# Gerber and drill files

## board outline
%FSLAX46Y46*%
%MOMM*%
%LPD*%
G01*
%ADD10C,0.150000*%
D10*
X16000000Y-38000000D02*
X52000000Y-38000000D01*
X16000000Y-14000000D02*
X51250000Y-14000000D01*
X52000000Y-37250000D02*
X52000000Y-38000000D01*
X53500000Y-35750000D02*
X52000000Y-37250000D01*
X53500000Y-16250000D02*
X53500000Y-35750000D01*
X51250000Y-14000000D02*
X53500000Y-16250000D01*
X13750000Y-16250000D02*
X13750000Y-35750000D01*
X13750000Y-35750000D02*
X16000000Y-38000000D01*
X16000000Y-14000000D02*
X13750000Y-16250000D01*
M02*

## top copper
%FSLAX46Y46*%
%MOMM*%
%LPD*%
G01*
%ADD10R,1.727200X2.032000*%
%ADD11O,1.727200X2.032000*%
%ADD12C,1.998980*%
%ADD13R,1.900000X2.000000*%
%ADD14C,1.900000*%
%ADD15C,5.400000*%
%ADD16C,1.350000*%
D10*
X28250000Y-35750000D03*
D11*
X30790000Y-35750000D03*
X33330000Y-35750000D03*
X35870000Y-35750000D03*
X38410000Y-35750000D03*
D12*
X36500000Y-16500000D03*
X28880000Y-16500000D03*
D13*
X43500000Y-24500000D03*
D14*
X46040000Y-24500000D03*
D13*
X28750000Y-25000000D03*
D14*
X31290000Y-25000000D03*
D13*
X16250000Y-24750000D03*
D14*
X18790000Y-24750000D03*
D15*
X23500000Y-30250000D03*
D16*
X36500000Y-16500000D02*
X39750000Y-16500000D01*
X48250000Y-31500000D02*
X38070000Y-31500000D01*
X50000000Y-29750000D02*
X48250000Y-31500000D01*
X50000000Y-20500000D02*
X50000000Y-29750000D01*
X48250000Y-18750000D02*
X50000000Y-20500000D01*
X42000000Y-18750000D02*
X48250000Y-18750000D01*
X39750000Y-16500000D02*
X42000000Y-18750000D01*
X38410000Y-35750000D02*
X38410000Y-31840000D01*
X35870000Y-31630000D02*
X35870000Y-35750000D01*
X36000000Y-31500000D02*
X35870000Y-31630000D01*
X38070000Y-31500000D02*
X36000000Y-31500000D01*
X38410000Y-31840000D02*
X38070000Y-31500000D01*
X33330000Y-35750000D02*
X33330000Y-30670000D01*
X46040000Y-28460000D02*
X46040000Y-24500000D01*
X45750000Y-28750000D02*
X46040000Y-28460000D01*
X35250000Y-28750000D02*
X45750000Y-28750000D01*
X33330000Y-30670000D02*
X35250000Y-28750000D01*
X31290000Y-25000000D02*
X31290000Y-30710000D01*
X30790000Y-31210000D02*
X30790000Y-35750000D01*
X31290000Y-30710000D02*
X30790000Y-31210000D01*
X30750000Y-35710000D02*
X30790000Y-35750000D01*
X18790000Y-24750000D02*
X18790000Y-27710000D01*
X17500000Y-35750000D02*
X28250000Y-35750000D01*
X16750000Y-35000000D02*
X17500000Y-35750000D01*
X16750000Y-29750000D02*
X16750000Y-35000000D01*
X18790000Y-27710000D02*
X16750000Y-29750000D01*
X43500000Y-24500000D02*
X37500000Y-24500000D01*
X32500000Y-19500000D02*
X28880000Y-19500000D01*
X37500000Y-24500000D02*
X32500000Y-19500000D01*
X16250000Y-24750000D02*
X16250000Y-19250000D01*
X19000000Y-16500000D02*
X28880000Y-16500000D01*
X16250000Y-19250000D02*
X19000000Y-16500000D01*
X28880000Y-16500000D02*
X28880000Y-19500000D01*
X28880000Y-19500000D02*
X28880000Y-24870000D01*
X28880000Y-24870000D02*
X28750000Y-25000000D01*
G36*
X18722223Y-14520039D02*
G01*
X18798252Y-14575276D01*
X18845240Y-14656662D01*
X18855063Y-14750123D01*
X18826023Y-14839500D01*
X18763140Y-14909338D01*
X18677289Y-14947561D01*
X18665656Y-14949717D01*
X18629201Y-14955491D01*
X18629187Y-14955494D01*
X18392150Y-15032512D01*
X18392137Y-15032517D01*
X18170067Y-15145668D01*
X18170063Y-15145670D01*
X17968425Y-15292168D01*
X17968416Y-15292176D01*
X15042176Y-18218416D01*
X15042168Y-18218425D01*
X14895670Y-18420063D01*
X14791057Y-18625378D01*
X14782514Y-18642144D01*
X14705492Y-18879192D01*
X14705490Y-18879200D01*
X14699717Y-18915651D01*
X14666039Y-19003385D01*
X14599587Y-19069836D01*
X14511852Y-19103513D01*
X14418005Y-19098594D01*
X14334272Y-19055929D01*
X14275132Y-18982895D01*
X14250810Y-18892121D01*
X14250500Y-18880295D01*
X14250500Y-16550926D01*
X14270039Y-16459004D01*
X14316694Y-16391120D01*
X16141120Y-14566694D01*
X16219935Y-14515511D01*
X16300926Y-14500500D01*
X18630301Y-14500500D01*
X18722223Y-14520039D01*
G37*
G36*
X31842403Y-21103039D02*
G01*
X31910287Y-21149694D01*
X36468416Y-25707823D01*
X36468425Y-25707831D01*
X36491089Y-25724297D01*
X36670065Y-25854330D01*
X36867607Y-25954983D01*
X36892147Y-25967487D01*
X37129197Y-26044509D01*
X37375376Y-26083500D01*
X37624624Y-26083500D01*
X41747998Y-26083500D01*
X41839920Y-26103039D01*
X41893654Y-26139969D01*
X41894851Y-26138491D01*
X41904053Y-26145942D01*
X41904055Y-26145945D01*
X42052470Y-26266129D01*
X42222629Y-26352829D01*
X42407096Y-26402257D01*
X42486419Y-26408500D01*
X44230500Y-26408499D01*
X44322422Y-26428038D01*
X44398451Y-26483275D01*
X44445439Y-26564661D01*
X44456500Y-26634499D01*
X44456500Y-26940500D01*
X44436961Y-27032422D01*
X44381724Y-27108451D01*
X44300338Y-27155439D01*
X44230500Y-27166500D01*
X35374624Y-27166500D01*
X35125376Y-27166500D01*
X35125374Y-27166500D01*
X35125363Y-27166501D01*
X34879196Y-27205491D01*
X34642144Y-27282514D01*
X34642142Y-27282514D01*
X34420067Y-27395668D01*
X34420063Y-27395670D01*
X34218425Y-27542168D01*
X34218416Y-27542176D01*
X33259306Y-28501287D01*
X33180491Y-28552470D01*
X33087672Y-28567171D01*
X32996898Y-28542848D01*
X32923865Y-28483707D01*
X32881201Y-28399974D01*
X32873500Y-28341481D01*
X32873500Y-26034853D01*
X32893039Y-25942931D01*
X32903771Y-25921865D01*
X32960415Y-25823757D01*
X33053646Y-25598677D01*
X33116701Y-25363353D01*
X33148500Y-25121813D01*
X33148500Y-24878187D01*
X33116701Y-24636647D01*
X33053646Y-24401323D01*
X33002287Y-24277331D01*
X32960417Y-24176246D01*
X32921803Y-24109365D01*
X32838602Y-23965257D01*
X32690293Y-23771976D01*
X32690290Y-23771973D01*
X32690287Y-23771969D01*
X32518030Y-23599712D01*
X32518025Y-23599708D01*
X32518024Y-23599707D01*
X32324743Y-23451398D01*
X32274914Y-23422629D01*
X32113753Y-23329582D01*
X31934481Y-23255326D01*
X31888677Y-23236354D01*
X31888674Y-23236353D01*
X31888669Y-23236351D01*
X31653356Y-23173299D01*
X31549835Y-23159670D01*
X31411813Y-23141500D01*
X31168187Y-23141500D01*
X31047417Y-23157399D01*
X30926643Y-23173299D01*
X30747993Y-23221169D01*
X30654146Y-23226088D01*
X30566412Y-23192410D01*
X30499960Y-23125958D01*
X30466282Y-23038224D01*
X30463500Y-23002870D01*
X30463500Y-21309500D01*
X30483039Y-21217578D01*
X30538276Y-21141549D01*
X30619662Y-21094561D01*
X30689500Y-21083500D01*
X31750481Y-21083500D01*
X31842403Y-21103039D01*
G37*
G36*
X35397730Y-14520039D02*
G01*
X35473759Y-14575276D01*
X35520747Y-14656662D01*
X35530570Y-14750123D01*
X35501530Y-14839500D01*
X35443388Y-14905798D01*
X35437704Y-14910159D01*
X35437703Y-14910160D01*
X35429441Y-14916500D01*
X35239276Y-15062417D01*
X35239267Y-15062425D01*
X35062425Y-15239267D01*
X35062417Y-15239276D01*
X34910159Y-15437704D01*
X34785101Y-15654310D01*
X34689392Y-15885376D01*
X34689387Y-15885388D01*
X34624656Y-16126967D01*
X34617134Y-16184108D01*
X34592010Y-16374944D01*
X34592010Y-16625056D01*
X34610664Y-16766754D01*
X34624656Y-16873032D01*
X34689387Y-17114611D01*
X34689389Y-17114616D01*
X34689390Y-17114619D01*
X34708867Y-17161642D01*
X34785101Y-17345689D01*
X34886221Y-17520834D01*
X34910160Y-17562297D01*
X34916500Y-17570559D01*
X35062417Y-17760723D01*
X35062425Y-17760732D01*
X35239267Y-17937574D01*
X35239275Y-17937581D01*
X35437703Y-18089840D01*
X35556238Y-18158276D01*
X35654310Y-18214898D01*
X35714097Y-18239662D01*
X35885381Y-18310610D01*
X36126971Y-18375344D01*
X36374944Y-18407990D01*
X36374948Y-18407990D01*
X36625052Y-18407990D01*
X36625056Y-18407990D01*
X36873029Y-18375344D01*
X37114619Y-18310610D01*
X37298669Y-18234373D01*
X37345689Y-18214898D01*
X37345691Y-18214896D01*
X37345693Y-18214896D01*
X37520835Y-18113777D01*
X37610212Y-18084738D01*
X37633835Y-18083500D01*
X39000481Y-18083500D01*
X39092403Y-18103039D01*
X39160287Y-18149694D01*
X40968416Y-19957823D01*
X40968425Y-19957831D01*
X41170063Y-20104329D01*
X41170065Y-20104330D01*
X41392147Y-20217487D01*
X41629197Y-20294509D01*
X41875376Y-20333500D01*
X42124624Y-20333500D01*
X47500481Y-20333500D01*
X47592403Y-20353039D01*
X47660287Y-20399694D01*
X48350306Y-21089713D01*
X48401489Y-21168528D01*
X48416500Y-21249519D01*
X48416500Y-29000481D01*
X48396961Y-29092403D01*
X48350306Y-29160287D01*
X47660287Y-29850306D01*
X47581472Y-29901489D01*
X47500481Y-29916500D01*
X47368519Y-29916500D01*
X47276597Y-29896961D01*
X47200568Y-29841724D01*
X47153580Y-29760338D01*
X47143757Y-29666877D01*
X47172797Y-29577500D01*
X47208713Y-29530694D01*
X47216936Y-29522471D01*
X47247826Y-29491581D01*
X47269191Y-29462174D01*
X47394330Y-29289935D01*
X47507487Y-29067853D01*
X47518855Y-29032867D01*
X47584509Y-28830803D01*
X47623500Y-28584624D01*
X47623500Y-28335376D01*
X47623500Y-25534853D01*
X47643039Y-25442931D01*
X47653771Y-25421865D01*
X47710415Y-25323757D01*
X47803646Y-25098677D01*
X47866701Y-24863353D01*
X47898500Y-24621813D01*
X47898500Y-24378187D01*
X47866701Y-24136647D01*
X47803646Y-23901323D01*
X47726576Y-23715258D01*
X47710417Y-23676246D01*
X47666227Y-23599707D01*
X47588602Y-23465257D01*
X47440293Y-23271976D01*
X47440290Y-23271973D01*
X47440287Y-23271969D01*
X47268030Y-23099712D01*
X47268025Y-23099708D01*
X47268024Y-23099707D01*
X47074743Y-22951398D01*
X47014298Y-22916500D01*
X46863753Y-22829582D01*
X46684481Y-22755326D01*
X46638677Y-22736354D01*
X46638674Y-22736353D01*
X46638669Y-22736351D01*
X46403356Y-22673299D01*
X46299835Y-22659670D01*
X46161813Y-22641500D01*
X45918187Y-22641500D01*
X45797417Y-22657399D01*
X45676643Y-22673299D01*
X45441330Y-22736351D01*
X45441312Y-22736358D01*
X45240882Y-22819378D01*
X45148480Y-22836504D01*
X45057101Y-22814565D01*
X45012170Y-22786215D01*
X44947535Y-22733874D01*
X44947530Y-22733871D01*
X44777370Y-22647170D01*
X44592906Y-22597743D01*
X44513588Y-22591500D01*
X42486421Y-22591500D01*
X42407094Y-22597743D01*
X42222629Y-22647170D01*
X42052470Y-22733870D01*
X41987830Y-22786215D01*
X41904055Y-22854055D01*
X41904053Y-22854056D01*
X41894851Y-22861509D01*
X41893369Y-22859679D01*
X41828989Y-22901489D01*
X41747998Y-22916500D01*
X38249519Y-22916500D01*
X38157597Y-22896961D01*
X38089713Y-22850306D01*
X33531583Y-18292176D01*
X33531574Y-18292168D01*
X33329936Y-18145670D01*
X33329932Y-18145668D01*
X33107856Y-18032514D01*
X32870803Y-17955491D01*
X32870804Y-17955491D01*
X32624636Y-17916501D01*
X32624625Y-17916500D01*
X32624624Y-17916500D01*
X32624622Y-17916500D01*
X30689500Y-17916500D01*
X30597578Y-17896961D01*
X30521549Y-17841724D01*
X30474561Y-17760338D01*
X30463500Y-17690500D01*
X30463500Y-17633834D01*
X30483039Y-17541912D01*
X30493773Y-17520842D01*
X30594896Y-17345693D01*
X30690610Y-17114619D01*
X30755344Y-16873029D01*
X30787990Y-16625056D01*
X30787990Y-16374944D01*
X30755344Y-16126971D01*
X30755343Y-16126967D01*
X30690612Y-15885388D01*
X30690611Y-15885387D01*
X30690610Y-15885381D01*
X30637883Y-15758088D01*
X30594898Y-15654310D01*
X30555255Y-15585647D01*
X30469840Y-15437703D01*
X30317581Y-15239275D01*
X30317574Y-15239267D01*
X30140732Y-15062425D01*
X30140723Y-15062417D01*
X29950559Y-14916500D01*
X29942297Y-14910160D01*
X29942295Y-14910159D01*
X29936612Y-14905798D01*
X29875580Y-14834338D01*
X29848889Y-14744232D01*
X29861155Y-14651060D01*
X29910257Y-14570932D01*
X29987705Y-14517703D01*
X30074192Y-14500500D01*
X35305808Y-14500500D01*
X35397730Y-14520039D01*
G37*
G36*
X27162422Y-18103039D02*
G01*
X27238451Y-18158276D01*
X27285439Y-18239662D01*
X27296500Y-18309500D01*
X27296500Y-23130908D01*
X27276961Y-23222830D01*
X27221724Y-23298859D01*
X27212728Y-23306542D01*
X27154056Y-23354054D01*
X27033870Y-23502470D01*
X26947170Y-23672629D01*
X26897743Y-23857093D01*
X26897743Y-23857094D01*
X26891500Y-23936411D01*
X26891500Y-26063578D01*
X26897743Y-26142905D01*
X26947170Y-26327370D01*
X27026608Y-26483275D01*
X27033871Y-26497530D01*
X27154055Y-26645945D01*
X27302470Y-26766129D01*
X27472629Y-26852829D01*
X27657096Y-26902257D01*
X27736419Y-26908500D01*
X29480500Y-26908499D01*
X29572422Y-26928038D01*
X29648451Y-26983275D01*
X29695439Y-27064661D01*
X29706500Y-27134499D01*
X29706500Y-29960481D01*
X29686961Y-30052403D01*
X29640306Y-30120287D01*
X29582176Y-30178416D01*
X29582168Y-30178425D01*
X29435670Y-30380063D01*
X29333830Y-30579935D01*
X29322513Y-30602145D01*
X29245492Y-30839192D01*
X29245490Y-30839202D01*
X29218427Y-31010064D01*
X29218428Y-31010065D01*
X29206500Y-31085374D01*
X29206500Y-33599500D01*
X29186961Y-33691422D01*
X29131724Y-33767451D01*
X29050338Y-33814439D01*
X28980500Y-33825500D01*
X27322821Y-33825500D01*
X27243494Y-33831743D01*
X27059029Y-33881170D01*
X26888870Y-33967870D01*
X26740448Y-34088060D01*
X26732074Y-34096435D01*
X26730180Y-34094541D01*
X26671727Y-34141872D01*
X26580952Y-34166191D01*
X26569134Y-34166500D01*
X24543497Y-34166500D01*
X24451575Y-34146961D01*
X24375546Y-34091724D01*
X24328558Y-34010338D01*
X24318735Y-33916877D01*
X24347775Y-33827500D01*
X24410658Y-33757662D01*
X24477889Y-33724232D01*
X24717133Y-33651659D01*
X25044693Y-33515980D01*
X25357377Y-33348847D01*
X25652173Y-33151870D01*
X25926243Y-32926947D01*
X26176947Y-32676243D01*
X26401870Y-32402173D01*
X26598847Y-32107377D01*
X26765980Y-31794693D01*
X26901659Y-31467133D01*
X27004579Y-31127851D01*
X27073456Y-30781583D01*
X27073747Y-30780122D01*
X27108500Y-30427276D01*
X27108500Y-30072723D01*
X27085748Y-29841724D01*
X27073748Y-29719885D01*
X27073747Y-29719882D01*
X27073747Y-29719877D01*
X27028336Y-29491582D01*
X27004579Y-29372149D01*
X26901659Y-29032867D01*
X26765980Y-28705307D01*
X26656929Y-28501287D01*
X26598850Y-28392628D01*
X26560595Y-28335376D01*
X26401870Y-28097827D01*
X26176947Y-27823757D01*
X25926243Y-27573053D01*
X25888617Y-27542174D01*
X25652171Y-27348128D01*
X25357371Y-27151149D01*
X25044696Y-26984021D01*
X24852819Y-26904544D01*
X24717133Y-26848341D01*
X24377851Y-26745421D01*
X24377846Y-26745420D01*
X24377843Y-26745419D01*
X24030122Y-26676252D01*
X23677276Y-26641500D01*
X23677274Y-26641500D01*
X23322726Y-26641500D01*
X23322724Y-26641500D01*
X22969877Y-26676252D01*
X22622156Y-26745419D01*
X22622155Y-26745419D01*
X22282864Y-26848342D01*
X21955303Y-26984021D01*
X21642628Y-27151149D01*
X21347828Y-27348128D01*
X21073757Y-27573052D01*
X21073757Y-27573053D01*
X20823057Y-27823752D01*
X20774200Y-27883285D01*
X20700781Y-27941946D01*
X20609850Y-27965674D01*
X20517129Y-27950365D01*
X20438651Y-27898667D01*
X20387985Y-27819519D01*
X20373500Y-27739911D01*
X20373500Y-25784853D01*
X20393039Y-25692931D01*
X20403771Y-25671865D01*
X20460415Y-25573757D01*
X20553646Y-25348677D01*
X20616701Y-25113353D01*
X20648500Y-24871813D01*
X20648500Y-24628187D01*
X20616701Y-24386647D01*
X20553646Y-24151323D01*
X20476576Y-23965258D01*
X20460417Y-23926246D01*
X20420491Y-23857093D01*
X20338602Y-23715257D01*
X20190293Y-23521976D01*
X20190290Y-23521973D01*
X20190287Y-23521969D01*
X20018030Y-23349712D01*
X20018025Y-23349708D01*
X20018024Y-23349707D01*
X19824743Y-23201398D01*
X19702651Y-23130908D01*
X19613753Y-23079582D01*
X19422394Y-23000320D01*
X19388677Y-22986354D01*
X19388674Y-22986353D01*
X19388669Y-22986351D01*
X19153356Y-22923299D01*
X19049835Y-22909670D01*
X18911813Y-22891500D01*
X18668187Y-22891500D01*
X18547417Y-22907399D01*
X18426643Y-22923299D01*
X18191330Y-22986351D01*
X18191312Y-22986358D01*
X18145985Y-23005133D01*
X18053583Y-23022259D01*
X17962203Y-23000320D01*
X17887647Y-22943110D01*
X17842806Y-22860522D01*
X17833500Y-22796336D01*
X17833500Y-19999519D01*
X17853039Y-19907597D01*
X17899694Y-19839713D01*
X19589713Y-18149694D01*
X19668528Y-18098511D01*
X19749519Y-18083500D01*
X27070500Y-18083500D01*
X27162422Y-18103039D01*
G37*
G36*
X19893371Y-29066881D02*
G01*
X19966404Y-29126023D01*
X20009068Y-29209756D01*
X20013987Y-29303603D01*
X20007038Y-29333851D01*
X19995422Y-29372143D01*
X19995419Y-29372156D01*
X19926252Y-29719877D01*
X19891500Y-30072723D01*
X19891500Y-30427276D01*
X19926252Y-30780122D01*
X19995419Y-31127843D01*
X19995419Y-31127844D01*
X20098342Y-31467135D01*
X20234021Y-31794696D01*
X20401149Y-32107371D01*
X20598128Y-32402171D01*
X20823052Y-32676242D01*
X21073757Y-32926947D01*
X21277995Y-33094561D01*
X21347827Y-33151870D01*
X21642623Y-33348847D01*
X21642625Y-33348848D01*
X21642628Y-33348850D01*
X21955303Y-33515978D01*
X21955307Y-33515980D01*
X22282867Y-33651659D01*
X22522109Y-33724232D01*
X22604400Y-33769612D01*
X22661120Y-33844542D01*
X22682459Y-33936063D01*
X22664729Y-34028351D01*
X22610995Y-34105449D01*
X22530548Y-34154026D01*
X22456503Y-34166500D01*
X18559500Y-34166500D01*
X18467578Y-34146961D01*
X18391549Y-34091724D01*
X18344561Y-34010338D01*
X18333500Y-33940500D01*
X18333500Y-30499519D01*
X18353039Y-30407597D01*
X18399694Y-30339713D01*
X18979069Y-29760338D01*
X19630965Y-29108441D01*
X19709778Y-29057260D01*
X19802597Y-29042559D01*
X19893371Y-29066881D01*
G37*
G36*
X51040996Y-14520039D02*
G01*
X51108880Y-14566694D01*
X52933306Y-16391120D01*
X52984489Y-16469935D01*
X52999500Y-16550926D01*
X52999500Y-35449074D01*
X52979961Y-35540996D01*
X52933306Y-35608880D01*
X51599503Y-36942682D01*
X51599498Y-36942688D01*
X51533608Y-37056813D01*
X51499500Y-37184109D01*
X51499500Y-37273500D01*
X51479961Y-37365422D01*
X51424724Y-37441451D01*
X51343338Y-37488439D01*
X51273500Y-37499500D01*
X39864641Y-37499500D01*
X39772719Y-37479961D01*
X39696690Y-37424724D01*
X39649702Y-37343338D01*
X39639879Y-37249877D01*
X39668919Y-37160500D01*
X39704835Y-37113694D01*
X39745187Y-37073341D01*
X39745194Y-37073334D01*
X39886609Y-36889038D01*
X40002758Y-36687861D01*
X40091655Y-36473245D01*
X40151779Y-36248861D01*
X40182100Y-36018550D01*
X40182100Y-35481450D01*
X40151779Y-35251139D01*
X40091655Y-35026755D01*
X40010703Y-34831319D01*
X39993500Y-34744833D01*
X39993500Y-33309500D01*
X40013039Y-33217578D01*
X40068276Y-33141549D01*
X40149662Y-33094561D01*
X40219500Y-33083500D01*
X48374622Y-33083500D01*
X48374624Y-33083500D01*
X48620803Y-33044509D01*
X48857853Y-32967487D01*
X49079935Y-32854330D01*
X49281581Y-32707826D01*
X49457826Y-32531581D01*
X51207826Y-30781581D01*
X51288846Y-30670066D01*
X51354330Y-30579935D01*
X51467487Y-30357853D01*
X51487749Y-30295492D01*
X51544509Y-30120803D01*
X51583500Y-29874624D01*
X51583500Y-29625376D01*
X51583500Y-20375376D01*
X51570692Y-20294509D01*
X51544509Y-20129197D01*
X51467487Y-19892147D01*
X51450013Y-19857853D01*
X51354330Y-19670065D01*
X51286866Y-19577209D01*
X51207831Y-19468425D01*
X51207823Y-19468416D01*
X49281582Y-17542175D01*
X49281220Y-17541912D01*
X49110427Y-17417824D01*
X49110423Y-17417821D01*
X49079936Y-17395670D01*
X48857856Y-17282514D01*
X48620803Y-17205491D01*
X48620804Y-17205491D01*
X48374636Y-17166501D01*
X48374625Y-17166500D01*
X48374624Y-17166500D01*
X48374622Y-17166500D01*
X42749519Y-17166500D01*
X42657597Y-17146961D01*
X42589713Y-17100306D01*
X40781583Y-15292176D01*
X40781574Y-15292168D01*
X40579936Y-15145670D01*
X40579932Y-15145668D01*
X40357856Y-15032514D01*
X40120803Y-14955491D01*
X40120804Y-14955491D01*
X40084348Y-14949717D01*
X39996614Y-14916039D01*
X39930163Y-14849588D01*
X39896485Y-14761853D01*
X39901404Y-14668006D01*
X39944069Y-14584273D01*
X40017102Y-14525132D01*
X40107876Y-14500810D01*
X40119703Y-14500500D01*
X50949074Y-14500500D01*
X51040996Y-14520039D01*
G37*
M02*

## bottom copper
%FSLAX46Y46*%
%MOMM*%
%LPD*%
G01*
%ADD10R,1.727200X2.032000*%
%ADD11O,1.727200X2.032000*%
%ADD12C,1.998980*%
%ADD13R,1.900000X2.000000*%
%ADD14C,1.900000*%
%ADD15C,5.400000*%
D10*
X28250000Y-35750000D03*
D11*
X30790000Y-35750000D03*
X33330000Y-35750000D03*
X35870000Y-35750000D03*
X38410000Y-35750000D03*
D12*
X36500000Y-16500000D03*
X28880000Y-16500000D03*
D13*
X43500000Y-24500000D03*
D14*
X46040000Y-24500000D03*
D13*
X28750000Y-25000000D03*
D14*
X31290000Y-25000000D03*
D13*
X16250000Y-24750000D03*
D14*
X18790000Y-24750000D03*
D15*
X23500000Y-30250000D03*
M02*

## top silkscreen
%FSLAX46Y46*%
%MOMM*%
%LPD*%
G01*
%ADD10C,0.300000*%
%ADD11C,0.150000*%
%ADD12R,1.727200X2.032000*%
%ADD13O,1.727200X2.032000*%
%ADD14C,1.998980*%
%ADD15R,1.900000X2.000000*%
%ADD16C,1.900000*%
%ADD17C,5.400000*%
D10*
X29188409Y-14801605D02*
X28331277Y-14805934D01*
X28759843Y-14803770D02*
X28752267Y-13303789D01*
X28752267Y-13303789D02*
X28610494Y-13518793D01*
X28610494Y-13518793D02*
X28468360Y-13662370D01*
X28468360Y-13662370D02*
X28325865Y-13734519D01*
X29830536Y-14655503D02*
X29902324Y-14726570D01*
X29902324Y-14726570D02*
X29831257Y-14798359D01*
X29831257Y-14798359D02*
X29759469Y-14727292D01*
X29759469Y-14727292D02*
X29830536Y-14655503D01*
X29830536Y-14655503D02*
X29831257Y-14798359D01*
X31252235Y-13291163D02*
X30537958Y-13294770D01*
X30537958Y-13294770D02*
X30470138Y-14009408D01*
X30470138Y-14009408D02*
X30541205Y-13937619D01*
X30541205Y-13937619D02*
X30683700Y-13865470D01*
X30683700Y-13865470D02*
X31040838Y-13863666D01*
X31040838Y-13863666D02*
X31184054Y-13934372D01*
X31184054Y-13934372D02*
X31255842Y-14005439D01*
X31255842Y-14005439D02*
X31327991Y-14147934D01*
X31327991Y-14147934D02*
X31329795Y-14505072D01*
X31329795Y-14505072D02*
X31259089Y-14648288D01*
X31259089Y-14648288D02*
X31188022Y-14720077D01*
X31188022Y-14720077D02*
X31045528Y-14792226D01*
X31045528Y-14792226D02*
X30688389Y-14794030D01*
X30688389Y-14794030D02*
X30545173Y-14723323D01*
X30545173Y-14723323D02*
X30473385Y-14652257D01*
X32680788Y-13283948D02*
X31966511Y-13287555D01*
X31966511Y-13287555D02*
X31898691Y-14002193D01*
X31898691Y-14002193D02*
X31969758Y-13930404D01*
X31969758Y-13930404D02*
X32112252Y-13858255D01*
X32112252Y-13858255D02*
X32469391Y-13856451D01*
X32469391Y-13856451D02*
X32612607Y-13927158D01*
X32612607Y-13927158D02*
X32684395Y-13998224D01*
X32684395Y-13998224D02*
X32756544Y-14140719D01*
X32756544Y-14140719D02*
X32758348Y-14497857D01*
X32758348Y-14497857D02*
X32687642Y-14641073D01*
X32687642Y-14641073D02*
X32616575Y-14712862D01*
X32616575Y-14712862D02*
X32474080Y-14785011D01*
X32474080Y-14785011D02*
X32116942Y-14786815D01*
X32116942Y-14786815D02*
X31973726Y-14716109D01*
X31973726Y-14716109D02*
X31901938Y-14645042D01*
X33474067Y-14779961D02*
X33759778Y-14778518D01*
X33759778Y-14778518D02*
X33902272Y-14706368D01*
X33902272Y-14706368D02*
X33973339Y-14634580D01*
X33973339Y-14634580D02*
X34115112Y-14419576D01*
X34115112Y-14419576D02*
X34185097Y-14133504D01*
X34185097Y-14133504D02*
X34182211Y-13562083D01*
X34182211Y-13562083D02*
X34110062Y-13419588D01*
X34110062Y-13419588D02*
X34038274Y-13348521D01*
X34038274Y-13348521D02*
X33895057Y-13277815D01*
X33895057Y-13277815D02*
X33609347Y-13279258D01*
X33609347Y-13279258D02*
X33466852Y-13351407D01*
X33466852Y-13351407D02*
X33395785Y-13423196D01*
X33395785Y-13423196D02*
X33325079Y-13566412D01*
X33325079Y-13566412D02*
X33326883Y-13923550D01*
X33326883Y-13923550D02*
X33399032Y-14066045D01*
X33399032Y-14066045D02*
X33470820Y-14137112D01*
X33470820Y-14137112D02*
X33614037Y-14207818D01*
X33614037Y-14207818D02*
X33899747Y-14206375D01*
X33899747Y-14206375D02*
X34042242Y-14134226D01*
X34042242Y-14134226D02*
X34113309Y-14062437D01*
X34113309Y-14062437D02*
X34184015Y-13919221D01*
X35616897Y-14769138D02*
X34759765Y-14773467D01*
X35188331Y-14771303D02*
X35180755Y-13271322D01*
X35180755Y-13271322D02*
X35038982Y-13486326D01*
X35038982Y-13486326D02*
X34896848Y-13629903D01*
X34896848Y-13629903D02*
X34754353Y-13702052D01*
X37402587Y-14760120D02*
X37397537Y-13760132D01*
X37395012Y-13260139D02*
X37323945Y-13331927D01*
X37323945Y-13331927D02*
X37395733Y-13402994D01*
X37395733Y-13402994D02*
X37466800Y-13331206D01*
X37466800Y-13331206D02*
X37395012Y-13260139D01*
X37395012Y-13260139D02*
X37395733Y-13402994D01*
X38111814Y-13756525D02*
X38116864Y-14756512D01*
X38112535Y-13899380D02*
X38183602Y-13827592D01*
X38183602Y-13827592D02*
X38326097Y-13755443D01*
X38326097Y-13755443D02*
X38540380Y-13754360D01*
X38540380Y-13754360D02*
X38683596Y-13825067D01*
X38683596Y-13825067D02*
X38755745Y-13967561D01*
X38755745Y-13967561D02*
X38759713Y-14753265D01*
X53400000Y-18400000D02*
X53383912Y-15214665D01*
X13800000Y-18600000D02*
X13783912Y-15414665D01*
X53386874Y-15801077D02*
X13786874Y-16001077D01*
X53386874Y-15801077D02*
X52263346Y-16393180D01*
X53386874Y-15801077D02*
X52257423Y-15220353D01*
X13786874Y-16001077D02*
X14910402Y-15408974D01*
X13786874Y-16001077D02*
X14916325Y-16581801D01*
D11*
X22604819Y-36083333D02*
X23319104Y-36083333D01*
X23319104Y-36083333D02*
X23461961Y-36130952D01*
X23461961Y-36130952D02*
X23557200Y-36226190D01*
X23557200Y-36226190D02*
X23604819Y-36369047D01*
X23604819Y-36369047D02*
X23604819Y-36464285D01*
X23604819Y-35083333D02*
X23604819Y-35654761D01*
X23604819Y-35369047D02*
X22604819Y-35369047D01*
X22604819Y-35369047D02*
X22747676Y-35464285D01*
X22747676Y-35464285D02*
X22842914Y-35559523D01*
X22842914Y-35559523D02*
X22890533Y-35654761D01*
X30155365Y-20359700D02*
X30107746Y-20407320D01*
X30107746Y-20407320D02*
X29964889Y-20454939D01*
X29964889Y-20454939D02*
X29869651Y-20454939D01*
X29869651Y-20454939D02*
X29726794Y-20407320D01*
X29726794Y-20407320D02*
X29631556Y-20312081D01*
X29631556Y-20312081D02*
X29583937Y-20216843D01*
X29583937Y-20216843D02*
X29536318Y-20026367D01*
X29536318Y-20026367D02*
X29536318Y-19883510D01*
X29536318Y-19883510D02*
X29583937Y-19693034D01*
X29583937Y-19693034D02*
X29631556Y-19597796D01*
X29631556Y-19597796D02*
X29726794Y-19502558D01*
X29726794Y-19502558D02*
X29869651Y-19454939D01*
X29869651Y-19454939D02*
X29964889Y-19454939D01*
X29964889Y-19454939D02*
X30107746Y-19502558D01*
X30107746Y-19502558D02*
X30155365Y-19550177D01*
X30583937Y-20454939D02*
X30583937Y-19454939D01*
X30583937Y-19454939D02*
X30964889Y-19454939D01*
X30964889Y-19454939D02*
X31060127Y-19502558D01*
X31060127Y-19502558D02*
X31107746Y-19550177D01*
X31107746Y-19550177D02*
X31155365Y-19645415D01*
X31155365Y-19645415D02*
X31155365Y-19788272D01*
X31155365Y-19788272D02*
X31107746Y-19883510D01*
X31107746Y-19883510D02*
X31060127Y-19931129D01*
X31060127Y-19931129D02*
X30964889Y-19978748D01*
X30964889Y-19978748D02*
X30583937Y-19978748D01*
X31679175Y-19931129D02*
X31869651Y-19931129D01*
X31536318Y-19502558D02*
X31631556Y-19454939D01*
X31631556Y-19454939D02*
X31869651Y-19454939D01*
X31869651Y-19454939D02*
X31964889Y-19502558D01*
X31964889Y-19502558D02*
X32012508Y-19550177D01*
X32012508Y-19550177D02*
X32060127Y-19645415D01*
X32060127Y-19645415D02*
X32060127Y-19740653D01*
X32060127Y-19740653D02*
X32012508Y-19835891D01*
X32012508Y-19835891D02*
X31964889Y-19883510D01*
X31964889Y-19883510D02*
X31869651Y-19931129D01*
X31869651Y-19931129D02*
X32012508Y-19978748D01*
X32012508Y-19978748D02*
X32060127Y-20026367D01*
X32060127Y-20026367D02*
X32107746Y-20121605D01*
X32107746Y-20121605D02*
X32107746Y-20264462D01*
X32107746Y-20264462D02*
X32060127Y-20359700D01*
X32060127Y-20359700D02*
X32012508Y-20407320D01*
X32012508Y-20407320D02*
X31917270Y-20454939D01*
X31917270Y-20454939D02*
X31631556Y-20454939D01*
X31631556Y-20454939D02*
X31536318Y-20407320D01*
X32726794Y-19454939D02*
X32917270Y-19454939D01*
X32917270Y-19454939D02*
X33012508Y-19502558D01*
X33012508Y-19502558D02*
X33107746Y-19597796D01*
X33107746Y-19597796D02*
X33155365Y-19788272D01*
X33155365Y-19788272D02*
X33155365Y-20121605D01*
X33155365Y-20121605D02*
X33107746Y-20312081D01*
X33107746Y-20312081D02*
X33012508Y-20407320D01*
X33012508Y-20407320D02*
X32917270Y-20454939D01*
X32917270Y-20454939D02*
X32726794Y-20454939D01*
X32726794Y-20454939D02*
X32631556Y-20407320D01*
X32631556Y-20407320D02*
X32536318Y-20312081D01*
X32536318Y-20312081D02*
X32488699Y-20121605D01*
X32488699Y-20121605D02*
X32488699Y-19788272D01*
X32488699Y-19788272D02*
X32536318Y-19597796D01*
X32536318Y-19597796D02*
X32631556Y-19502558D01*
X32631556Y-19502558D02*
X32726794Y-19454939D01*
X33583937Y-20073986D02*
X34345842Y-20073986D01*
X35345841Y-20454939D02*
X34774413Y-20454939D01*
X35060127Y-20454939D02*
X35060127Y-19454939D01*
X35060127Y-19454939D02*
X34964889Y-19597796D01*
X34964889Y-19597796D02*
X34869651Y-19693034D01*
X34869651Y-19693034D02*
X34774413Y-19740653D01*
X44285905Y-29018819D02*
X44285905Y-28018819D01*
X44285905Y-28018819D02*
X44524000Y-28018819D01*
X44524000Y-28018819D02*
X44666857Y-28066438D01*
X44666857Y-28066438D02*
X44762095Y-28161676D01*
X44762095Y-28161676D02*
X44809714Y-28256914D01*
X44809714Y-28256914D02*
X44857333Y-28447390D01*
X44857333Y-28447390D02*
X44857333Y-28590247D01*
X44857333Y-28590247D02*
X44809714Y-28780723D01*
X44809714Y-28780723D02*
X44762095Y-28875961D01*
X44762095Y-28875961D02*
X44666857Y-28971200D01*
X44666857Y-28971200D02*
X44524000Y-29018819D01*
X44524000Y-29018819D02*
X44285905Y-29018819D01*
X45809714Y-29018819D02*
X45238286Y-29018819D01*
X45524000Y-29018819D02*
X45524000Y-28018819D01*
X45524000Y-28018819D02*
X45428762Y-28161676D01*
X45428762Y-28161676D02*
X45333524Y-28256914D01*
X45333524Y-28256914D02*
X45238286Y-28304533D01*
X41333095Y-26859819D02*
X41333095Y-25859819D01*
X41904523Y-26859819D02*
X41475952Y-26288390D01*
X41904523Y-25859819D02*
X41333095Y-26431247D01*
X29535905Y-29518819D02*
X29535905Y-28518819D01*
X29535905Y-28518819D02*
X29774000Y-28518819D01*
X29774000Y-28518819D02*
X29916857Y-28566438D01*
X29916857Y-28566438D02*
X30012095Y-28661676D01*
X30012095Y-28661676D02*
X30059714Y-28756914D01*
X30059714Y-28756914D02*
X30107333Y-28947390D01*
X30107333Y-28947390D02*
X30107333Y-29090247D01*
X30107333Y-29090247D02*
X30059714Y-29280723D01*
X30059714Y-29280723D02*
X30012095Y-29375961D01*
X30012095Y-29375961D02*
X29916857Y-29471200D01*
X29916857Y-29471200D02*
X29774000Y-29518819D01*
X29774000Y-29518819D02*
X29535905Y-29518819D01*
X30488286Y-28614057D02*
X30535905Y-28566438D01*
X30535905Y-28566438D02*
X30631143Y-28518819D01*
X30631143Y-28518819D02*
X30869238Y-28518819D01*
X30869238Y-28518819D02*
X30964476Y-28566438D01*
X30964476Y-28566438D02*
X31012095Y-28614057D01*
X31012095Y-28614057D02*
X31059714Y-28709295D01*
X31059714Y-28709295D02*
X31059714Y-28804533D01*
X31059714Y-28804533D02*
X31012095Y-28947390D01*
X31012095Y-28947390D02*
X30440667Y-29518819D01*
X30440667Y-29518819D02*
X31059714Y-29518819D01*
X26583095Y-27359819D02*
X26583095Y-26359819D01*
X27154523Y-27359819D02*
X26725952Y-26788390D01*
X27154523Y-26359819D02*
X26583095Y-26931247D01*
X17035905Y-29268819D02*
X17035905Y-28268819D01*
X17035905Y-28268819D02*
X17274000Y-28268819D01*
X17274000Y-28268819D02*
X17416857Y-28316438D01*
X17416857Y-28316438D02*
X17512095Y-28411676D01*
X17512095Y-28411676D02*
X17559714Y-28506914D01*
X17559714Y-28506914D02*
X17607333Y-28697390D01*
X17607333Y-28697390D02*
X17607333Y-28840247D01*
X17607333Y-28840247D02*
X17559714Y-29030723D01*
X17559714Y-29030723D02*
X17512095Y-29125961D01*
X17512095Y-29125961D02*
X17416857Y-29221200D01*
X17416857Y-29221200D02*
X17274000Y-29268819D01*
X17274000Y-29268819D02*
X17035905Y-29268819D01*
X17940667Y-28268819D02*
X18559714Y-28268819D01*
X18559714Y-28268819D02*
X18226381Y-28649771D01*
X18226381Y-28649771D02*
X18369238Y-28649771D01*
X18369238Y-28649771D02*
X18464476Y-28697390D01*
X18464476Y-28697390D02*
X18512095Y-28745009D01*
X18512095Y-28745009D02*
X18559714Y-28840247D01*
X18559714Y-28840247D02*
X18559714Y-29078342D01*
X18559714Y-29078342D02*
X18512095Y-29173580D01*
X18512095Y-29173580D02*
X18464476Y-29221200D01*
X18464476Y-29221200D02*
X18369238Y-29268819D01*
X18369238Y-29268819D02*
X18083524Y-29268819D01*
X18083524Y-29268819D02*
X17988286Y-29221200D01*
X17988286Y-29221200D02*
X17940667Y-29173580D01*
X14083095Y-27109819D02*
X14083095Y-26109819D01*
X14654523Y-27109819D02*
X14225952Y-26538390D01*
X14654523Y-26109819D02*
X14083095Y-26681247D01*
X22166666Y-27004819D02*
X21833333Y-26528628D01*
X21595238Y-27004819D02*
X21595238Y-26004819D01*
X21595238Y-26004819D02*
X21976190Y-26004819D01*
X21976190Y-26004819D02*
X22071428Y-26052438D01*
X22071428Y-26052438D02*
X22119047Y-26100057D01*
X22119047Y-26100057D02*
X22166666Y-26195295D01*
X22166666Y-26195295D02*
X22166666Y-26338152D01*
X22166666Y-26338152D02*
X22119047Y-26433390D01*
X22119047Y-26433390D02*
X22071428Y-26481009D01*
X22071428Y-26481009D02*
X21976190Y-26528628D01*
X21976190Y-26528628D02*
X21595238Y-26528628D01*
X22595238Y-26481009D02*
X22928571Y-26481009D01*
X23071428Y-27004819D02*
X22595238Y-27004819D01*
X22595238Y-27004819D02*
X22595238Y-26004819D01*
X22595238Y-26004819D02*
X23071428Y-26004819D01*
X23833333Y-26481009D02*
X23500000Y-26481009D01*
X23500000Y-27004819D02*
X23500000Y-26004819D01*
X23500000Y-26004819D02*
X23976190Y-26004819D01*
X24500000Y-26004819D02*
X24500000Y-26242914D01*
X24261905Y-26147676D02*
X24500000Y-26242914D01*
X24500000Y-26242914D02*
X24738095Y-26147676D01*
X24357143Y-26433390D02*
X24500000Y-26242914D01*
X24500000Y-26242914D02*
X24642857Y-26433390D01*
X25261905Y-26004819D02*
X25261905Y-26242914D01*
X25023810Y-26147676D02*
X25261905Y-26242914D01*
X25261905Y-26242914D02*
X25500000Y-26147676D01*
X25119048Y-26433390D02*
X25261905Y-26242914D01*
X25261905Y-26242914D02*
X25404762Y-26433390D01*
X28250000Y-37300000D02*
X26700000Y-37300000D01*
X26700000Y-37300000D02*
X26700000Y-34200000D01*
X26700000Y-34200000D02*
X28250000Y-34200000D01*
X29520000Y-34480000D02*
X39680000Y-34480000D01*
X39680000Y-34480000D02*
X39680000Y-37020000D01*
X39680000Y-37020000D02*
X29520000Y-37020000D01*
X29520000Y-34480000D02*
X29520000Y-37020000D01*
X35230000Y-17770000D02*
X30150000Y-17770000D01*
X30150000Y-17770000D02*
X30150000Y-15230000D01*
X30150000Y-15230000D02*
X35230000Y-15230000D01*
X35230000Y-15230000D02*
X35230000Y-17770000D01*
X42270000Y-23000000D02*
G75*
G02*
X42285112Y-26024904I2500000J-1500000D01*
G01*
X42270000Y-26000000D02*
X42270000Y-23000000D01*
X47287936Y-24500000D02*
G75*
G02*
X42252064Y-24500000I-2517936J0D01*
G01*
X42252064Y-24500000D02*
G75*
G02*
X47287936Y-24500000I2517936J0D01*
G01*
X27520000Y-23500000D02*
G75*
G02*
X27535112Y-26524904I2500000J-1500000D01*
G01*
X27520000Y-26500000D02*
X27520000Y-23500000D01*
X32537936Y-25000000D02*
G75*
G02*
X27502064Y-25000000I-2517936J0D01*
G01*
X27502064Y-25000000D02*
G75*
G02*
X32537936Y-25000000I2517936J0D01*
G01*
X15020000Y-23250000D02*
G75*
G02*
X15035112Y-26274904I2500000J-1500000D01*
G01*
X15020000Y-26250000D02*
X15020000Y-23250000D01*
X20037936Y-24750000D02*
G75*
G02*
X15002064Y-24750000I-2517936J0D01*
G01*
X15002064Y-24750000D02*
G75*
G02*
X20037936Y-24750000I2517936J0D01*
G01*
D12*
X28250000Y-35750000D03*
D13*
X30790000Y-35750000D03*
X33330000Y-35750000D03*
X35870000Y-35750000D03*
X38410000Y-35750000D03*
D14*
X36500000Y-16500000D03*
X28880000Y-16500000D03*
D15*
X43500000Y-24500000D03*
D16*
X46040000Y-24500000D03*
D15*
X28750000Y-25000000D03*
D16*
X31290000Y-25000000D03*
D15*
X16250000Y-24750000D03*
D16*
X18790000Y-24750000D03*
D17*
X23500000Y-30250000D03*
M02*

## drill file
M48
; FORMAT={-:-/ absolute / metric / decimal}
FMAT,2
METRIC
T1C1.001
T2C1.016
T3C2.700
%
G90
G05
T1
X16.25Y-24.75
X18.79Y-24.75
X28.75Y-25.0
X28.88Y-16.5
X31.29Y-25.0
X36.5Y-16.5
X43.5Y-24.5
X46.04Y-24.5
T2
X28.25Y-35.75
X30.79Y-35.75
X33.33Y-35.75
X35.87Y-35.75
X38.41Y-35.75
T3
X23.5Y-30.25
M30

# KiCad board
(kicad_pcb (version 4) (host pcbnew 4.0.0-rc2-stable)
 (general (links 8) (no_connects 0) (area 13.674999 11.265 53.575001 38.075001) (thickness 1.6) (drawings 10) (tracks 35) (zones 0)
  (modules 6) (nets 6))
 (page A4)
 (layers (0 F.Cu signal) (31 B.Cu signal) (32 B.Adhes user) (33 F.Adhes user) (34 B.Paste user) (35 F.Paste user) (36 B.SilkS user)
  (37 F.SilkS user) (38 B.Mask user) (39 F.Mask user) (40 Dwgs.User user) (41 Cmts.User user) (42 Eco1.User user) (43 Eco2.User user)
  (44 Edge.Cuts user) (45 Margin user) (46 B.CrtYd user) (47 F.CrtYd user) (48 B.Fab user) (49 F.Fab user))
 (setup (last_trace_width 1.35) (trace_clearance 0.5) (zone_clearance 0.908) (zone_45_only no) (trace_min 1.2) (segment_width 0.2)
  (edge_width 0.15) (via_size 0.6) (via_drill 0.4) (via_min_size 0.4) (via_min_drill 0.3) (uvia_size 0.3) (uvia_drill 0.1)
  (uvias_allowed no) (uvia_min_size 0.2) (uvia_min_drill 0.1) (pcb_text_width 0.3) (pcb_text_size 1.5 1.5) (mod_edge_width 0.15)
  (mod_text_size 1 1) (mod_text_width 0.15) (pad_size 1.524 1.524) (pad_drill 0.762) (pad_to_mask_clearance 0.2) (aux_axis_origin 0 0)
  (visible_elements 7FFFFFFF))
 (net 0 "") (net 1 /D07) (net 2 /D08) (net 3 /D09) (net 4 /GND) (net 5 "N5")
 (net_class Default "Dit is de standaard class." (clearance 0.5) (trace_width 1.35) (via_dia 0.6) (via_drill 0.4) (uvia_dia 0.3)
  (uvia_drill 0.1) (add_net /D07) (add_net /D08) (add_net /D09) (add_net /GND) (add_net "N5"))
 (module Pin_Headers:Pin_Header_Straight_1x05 (layer F.Cu) (at 28.25 35.75 90)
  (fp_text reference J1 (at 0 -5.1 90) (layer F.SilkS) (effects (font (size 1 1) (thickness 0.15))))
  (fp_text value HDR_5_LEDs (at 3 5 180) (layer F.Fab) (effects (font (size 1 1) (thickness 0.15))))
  (fp_line (start -1.55 0) (end -1.55 -1.55) (layer F.SilkS) (width 0.15))
  (fp_line (start -1.55 -1.55) (end 1.55 -1.55) (layer F.SilkS) (width 0.15))
  (fp_line (start 1.55 -1.55) (end 1.55 0) (layer F.SilkS) (width 0.15))
  (fp_line (start 1.27 1.27) (end 1.27 11.43) (layer F.SilkS) (width 0.15))
  (fp_line (start 1.27 11.43) (end -1.27 11.43) (layer F.SilkS) (width 0.15))
  (fp_line (start -1.27 11.43) (end -1.27 1.27) (layer F.SilkS) (width 0.15))
  (fp_line (start 1.27 1.27) (end -1.27 1.27) (layer F.SilkS) (width 0.15))
  (pad 1 thru_hole rect (at 0 0 90) (size 2.032 1.7272) (drill 1.016) (layers *.Cu *.Mask F.SilkS) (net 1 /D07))
  (pad 2 thru_hole oval (at 0 2.54 90) (size 2.032 1.7272) (drill 1.016) (layers *.Cu *.Mask F.SilkS) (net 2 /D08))
  (pad 3 thru_hole oval (at 0 5.08 90) (size 2.032 1.7272) (drill 1.016) (layers *.Cu *.Mask F.SilkS) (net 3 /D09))
  (pad 4 thru_hole oval (at 0 7.62 90) (size 2.032 1.7272) (drill 1.016) (layers *.Cu *.Mask F.SilkS) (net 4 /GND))
  (pad 5 thru_hole oval (at 0 10.16 90) (size 2.032 1.7272) (drill 1.016) (layers *.Cu *.Mask F.SilkS) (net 4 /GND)))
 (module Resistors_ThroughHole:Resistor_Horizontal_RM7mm (layer F.Cu) (at 36.5 16.5 180)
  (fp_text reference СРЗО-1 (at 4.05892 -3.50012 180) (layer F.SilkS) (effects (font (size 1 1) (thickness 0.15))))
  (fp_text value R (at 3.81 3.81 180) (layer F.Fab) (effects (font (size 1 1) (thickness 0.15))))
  (fp_line (start 1.27 -1.27) (end 6.35 -1.27) (layer F.SilkS) (width 0.15))
  (fp_line (start 6.35 -1.27) (end 6.35 1.27) (layer F.SilkS) (width 0.15))
  (fp_line (start 6.35 1.27) (end 1.27 1.27) (layer F.SilkS) (width 0.15))
  (fp_line (start 1.27 1.27) (end 1.27 -1.27) (layer F.SilkS) (width 0.15))
  (pad 1 thru_hole circle (at 0 0 180) (size 1.99898 1.99898) (drill 1.00076) (layers *.Cu *.SilkS *.Mask) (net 4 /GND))
  (pad 2 thru_hole circle (at 7.62 0 180) (size 1.99898 1.99898) (drill 1.00076) (layers *.Cu *.SilkS *.Mask) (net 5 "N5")))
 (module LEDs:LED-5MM (layer F.Cu) (at 43.5 24.5)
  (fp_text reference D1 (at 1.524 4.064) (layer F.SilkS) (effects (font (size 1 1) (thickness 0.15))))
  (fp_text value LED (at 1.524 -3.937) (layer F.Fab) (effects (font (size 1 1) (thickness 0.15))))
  (fp_arc (start 1.27 0) (end -1.23 -1.5) (angle 297.5) (layer F.SilkS) (width 0.15))
  (fp_line (start -1.23 1.5) (end -1.23 -1.5) (layer F.SilkS) (width 0.15))
  (fp_circle (center 1.27 0) (end 0.97 -2.5) (layer F.SilkS) (width 0.15))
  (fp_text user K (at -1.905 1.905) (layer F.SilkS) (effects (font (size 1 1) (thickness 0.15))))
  (pad 1 thru_hole rect (at 0 0 90) (size 2 1.9) (drill 1.00076) (layers *.Cu *.Mask F.SilkS) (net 5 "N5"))
  (pad 2 thru_hole circle (at 2.54 0) (size 1.9 1.9) (drill 1.00076) (layers *.Cu *.Mask F.SilkS) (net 3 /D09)))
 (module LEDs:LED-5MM (layer F.Cu) (at 28.75 25)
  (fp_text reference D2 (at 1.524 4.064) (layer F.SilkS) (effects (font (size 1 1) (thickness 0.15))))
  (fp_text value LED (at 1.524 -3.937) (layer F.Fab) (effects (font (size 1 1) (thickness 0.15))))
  (fp_arc (start 1.27 0) (end -1.23 -1.5) (angle 297.5) (layer F.SilkS) (width 0.15))
  (fp_line (start -1.23 1.5) (end -1.23 -1.5) (layer F.SilkS) (width 0.15))
  (fp_circle (center 1.27 0) (end 0.97 -2.5) (layer F.SilkS) (width 0.15))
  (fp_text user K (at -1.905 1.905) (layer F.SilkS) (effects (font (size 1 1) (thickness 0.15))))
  (pad 1 thru_hole rect (at 0 0 90) (size 2 1.9) (drill 1.00076) (layers *.Cu *.Mask F.SilkS) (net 5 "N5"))
  (pad 2 thru_hole circle (at 2.54 0) (size 1.9 1.9) (drill 1.00076) (layers *.Cu *.Mask F.SilkS) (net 2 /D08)))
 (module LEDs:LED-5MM (layer F.Cu) (at 16.25 24.75)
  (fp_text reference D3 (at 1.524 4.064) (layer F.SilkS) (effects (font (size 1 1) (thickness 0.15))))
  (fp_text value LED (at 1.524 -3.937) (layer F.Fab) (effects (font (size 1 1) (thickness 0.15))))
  (fp_arc (start 1.27 0) (end -1.23 -1.5) (angle 297.5) (layer F.SilkS) (width 0.15))
  (fp_line (start -1.23 1.5) (end -1.23 -1.5) (layer F.SilkS) (width 0.15))
  (fp_circle (center 1.27 0) (end 0.97 -2.5) (layer F.SilkS) (width 0.15))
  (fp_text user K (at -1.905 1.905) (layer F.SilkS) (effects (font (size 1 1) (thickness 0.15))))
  (pad 1 thru_hole rect (at 0 0 90) (size 2 1.9) (drill 1.00076) (layers *.Cu *.Mask F.SilkS) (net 5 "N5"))
  (pad 2 thru_hole circle (at 2.54 0) (size 1.9 1.9) (drill 1.00076) (layers *.Cu *.Mask F.SilkS) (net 1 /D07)))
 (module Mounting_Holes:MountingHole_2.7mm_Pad (layer F.Cu) (at 23.5 30.25)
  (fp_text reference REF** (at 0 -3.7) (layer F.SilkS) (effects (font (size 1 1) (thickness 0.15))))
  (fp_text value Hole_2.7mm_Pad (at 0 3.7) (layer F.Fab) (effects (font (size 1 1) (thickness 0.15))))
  (pad 1 thru_hole circle (at 0 0) (size 5.4 5.4) (drill 2.7) (layers *.Cu *.Mask F.SilkS)))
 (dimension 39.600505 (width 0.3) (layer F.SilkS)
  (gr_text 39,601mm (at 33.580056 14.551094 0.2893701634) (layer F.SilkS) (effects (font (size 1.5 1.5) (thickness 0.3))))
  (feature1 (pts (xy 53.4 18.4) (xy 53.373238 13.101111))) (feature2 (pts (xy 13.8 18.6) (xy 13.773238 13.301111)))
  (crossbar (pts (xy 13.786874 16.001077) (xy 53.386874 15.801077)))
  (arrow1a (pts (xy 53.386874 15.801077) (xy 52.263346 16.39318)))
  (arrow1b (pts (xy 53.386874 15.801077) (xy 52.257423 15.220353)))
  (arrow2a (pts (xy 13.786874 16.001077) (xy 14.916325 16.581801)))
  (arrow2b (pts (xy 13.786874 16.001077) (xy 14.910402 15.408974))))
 (gr_line (start 16 38) (end 52 38) (angle 90) (layer Edge.Cuts) (width 0.15))
 (gr_line (start 16 14) (end 51.25 14) (angle 90) (layer Edge.Cuts) (width 0.15))
 (gr_line (start 52 37.25) (end 52 38) (angle 90) (layer Edge.Cuts) (width 0.15))
 (gr_line (start 53.5 35.75) (end 52 37.25) (angle 90) (layer Edge.Cuts) (width 0.15))
 (gr_line (start 53.5 16.25) (end 53.5 35.75) (angle 90) (layer Edge.Cuts) (width 0.15))
 (gr_line (start 51.25 14) (end 53.5 16.25) (angle 90) (layer Edge.Cuts) (width 0.15))
 (gr_line (start 13.75 16.25) (end 13.75 35.75) (angle 90) (layer Edge.Cuts) (width 0.15))
 (gr_line (start 13.75 35.75) (end 16 38) (angle 90) (layer Edge.Cuts) (width 0.15))
 (gr_line (start 16 14) (end 13.75 16.25) (angle 90) (layer Edge.Cuts) (width 0.15))
 (segment (start 36.5 16.5) (end 39.75 16.5) (width 1.35) (layer F.Cu) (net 4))
 (segment (start 48.25 31.5) (end 38.07 31.5) (width 1.35) (layer F.Cu) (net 4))
 (segment (start 50 29.75) (end 48.25 31.5) (width 1.35) (layer F.Cu) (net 4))
 (segment (start 50 20.5) (end 50 29.75) (width 1.35) (layer F.Cu) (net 4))
 (segment (start 48.25 18.75) (end 50 20.5) (width 1.35) (layer F.Cu) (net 4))
 (segment (start 42 18.75) (end 48.25 18.75) (width 1.35) (layer F.Cu) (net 4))
 (segment (start 39.75 16.5) (end 42 18.75) (width 1.35) (layer F.Cu) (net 4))
 (segment (start 38.41 35.75) (end 38.41 31.84) (width 1.35) (layer F.Cu) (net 4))
 (segment (start 35.87 31.63) (end 35.87 35.75) (width 1.35) (layer F.Cu) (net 4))
 (segment (start 36 31.5) (end 35.87 31.63) (width 1.35) (layer F.Cu) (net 4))
 (segment (start 38.07 31.5) (end 36 31.5) (width 1.35) (layer F.Cu) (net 4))
 (segment (start 38.41 31.84) (end 38.07 31.5) (width 1.35) (layer F.Cu) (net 4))
 (segment (start 33.33 35.75) (end 33.33 30.67) (width 1.35) (layer F.Cu) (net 3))
 (segment (start 46.04 28.46) (end 46.04 24.5) (width 1.35) (layer F.Cu) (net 3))
 (segment (start 45.75 28.75) (end 46.04 28.46) (width 1.35) (layer F.Cu) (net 3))
 (segment (start 35.25 28.75) (end 45.75 28.75) (width 1.35) (layer F.Cu) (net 3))
 (segment (start 33.33 30.67) (end 35.25 28.75) (width 1.35) (layer F.Cu) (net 3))
 (segment (start 31.29 25) (end 31.29 30.71) (width 1.35) (layer F.Cu) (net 2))
 (segment (start 30.79 31.21) (end 30.79 35.75) (width 1.35) (layer F.Cu) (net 2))
 (segment (start 31.29 30.71) (end 30.79 31.21) (width 1.35) (layer F.Cu) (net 2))
 (segment (start 30.75 35.71) (end 30.79 35.75) (width 1.35) (layer F.Cu) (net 2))
 (segment (start 18.79 24.75) (end 18.79 27.71) (width 1.35) (layer F.Cu) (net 1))
 (segment (start 17.5 35.75) (end 28.25 35.75) (width 1.35) (layer F.Cu) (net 1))
 (segment (start 16.75 35) (end 17.5 35.75) (width 1.35) (layer F.Cu) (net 1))
 (segment (start 16.75 29.75) (end 16.75 35) (width 1.35) (layer F.Cu) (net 1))
 (segment (start 18.79 27.71) (end 16.75 29.75) (width 1.35) (layer F.Cu) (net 1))
 (segment (start 43.5 24.5) (end 37.5 24.5) (width 1.35) (layer F.Cu) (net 5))
 (segment (start 32.5 19.5) (end 28.88 19.5) (width 1.35) (layer F.Cu) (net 5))
 (segment (start 37.5 24.5) (end 32.5 19.5) (width 1.35) (layer F.Cu) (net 5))
 (segment (start 16.25 24.75) (end 16.25 19.25) (width 1.35) (layer F.Cu) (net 5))
 (segment (start 19 16.5) (end 28.88 16.5) (width 1.35) (layer F.Cu) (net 5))
 (segment (start 16.25 19.25) (end 19 16.5) (width 1.35) (layer F.Cu) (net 5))
 (segment (start 28.88 16.5) (end 28.88 19.5) (width 1.35) (layer F.Cu) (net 5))
 (segment (start 28.88 19.5) (end 28.88 24.87) (width 1.35) (layer F.Cu) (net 5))
 (segment (start 28.88 24.87) (end 28.75 25) (width 1.35) (layer F.Cu) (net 5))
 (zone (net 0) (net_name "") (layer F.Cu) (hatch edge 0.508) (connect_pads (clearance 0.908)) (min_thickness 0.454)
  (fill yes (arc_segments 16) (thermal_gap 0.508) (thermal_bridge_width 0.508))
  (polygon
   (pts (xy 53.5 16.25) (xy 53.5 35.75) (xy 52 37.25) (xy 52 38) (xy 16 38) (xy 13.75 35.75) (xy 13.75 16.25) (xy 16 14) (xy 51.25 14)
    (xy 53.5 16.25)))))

